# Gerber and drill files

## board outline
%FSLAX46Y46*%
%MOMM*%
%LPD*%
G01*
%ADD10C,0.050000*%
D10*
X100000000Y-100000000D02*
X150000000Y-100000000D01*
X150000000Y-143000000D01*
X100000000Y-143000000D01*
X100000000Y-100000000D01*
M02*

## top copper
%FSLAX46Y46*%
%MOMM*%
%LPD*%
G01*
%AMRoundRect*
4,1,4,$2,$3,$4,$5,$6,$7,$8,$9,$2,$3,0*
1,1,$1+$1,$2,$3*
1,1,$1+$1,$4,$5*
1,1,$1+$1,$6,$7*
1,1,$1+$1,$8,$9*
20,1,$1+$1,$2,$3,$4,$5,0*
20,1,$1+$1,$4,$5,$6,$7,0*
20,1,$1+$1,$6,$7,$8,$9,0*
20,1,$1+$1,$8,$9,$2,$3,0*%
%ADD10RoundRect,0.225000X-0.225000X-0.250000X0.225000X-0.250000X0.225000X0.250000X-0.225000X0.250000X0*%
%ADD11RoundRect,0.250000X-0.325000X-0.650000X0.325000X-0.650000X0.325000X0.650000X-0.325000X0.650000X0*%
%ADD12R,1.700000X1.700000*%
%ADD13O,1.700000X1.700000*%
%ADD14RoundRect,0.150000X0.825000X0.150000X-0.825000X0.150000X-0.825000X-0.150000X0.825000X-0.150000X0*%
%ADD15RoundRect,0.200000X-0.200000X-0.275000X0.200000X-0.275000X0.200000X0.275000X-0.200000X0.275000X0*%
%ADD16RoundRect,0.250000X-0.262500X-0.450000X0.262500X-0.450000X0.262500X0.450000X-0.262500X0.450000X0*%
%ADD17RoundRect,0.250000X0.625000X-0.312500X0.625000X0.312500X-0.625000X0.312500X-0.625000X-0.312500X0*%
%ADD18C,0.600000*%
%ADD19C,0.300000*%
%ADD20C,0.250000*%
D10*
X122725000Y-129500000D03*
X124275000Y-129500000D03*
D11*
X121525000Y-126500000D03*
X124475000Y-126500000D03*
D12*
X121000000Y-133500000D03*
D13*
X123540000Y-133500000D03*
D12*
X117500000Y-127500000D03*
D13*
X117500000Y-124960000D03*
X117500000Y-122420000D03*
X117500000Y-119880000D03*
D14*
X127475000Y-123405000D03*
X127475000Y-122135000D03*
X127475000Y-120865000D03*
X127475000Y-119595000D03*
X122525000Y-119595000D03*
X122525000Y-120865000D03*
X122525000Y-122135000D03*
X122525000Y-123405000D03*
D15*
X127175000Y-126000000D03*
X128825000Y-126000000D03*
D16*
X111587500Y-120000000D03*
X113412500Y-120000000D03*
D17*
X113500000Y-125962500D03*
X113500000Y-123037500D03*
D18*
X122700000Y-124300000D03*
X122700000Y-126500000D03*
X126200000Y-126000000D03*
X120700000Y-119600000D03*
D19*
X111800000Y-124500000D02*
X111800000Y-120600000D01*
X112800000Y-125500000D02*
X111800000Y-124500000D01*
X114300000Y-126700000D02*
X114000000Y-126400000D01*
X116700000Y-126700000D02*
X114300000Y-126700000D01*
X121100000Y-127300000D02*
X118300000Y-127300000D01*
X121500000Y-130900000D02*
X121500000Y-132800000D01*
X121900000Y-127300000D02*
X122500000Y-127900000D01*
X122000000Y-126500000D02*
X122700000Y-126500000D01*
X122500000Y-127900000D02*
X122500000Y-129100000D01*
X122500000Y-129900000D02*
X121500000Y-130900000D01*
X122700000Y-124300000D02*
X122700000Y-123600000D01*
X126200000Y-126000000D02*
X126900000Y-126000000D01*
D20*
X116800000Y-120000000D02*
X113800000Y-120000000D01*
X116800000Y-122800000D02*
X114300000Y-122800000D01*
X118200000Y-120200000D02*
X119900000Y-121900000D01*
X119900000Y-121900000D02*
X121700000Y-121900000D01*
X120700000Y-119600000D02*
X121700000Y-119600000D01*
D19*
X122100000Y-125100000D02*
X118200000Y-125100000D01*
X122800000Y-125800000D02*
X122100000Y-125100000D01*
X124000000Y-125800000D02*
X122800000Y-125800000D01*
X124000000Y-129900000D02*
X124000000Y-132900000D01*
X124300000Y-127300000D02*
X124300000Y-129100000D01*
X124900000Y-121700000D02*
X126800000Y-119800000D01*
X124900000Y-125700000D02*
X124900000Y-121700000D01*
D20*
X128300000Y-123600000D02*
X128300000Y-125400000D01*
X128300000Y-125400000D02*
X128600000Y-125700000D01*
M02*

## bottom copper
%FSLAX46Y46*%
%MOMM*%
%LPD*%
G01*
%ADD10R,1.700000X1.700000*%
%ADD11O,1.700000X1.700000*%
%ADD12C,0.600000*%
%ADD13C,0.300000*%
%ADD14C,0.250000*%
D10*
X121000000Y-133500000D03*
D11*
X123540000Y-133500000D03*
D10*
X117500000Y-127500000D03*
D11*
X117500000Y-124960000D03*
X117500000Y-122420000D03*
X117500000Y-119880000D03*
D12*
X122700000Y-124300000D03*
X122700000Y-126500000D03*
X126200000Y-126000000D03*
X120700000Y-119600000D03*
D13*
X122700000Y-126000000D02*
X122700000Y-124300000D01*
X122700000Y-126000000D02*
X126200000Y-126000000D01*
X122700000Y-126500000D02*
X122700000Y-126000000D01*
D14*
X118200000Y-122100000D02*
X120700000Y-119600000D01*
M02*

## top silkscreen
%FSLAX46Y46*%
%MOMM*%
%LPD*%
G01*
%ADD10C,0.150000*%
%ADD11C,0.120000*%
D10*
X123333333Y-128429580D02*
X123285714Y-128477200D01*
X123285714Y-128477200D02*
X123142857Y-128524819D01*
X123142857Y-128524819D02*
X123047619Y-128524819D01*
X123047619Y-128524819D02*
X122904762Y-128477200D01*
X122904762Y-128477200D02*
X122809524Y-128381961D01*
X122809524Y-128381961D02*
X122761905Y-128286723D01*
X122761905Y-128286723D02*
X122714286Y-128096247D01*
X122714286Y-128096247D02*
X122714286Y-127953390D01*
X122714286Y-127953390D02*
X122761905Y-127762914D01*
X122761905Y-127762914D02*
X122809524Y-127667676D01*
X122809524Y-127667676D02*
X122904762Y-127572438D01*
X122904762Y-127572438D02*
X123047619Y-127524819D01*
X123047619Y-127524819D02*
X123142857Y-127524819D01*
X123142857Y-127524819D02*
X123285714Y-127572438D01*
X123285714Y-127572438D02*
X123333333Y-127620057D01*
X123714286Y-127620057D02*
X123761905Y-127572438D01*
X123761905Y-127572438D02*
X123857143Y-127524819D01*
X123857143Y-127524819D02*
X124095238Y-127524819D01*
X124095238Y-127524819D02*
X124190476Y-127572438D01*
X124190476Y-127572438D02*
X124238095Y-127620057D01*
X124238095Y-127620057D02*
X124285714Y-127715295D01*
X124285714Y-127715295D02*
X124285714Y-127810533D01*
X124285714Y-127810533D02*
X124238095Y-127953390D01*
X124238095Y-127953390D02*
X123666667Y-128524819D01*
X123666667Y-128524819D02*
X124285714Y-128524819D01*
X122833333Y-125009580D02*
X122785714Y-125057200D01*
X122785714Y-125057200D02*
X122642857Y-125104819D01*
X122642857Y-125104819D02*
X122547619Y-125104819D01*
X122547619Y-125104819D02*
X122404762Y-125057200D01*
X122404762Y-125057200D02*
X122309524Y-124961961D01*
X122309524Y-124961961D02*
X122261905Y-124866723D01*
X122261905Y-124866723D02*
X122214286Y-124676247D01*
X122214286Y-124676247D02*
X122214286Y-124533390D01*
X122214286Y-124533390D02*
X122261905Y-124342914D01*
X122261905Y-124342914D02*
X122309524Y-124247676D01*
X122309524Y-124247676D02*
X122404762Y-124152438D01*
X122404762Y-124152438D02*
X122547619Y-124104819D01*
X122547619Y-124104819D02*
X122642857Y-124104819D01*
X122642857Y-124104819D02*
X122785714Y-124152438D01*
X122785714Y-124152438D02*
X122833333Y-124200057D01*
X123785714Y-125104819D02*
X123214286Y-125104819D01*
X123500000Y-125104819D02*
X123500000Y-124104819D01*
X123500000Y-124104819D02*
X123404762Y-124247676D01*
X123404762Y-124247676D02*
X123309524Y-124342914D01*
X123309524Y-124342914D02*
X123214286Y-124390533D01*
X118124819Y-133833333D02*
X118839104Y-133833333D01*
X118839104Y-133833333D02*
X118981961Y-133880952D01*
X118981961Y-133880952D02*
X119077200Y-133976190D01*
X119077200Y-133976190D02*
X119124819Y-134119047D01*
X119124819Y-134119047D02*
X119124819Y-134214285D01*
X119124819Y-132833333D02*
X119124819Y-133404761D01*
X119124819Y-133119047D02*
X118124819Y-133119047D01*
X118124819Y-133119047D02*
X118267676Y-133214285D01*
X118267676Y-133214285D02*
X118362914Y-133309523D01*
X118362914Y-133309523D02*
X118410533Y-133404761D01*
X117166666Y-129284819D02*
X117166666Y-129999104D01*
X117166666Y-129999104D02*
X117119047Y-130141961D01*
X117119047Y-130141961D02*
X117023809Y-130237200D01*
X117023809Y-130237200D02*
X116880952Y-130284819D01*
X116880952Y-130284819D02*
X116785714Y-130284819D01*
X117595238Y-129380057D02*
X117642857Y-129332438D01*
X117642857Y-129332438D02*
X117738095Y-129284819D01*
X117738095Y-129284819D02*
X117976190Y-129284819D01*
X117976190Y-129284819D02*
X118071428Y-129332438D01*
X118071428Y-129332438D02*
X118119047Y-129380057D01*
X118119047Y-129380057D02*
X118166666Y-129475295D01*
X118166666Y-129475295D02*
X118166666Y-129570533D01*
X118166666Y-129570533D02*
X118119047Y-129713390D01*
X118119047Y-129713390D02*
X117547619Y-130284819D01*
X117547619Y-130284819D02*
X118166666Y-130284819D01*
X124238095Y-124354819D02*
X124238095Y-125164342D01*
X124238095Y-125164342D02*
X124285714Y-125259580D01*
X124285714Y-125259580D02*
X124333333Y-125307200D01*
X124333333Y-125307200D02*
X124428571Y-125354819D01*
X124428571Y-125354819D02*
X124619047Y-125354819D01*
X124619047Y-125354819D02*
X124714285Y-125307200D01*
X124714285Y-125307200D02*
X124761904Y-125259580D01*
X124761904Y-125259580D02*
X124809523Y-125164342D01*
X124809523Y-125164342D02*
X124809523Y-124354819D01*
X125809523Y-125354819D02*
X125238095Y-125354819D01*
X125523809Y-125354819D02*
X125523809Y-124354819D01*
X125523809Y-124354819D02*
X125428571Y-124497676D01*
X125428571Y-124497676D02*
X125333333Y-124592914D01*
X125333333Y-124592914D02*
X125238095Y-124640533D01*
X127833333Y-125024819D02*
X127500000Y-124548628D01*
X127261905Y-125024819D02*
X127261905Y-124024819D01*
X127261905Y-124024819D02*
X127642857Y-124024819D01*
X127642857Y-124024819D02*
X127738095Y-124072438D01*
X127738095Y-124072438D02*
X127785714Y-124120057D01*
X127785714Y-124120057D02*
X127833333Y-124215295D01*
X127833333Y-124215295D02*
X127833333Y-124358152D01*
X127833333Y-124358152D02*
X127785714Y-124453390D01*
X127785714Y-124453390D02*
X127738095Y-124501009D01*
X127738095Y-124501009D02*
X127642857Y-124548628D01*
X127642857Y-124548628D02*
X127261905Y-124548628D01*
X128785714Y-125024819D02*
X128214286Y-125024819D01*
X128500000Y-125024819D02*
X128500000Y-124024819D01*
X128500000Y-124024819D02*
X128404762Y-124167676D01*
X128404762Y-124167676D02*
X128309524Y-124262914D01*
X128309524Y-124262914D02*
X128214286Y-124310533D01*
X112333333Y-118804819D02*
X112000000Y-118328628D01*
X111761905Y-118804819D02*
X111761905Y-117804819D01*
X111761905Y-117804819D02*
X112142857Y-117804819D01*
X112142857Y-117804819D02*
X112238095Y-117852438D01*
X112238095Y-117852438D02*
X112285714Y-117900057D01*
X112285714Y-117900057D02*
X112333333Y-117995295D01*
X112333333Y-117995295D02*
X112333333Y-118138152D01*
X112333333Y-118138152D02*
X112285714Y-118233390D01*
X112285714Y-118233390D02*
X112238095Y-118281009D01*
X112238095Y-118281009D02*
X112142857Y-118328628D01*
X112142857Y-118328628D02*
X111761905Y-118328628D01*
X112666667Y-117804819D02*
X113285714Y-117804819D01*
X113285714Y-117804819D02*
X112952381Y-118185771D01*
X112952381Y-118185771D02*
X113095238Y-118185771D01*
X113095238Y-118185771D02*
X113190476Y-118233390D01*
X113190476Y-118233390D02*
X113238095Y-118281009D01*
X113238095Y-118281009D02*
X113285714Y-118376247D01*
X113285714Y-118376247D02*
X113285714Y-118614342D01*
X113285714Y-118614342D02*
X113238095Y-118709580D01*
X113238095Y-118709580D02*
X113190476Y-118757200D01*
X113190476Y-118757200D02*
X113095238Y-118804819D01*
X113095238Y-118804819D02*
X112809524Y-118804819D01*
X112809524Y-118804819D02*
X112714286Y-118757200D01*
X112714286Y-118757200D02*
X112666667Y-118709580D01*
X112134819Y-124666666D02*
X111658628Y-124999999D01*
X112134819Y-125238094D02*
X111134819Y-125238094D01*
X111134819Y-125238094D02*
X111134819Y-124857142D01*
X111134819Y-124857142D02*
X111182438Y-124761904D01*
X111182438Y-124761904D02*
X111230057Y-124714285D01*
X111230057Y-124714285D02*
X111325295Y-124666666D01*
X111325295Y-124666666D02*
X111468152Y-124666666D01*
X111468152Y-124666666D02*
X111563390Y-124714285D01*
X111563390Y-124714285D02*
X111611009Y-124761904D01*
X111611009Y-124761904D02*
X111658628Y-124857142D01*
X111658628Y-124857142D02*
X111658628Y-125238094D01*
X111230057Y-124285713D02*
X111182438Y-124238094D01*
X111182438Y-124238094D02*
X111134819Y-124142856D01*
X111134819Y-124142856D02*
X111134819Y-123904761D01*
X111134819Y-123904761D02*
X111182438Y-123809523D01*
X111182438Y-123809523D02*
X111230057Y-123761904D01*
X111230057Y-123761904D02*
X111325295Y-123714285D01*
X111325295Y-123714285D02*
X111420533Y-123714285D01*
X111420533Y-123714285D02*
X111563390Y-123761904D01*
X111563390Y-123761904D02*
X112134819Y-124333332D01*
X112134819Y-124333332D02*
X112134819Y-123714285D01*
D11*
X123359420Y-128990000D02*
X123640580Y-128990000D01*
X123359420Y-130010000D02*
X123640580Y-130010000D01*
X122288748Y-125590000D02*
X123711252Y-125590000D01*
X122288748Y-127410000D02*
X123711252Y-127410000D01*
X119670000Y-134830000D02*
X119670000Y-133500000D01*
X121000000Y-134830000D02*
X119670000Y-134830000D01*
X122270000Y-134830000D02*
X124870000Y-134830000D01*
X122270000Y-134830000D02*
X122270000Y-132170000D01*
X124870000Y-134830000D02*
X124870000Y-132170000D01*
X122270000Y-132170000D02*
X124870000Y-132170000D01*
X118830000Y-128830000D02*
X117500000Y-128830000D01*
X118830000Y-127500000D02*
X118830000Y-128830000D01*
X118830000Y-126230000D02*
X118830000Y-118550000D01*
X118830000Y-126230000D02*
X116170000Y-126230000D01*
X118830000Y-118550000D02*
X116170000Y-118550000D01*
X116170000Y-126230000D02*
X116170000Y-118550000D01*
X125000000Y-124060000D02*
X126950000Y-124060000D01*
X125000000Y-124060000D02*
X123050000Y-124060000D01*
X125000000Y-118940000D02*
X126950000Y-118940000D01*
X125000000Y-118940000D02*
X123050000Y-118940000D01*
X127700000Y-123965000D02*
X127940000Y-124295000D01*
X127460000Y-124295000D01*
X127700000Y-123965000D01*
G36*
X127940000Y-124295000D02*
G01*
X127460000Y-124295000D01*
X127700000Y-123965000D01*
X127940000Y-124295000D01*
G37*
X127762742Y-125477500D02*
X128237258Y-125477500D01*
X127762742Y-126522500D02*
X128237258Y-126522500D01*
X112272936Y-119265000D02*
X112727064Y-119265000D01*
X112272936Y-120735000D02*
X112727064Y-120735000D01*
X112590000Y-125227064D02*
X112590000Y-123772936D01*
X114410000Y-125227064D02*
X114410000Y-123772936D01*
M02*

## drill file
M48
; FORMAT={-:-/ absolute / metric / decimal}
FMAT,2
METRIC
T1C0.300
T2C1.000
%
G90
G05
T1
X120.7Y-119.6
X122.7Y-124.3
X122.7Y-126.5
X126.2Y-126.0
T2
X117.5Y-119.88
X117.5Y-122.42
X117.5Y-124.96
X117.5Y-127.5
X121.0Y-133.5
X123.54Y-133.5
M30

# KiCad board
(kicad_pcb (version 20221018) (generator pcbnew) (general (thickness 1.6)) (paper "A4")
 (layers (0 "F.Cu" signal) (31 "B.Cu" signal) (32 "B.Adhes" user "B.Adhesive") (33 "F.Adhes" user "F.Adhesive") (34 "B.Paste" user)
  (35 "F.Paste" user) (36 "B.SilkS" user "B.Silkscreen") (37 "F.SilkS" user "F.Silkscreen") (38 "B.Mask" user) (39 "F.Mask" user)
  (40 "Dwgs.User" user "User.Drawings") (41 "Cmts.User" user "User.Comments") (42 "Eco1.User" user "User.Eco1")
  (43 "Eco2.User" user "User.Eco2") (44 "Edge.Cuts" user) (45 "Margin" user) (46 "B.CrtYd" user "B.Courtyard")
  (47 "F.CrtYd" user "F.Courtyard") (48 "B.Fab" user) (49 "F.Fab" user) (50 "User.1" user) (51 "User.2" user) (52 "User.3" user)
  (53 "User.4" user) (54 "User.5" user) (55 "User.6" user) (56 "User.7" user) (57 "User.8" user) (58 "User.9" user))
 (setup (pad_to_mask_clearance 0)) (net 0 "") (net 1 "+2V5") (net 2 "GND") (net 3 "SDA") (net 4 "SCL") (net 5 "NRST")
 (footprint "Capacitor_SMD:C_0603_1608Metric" (layer "F.Cu") (at 123.5 129.5)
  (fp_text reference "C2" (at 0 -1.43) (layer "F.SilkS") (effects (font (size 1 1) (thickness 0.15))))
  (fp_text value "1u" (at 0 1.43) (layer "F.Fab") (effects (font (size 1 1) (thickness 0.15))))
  (fp_line (start -0.14058 -0.51) (end 0.14058 -0.51) (stroke (width 0.12) (type solid)) (layer "F.SilkS"))
  (fp_line (start -0.14058 0.51) (end 0.14058 0.51) (stroke (width 0.12) (type solid)) (layer "F.SilkS"))
  (pad "1" smd roundrect (at -0.775 0) (size 0.9 0.95) (layers "F.Cu" "F.Paste" "F.Mask") (roundrect_rratio 0.25) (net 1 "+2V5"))
  (pad "2" smd roundrect (at 0.775 0) (size 0.9 0.95) (layers "F.Cu" "F.Paste" "F.Mask") (roundrect_rratio 0.25) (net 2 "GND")))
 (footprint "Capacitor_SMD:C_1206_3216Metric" (layer "F.Cu") (at 123 126.5)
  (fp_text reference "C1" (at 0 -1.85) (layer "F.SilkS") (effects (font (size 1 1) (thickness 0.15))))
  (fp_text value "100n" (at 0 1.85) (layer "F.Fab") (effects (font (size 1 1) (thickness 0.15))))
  (fp_line (start -0.711252 -0.91) (end 0.711252 -0.91) (stroke (width 0.12) (type solid)) (layer "F.SilkS"))
  (fp_line (start -0.711252 0.91) (end 0.711252 0.91) (stroke (width 0.12) (type solid)) (layer "F.SilkS"))
  (pad "1" smd roundrect (at -1.475 0) (size 1.15 1.8) (layers "F.Cu" "F.Paste" "F.Mask") (roundrect_rratio 0.217391) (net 1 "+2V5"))
  (pad "2" smd roundrect (at 1.475 0) (size 1.15 1.8) (layers "F.Cu" "F.Paste" "F.Mask") (roundrect_rratio 0.217391) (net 2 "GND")))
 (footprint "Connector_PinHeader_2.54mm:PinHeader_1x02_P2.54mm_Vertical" (layer "F.Cu") (at 121 133.5 90)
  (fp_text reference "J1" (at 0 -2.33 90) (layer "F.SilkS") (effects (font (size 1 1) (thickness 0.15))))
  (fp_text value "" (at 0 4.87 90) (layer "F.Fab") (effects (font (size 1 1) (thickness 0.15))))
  (fp_line (start -1.33 -1.33) (end 0 -1.33) (stroke (width 0.12) (type solid)) (layer "F.SilkS"))
  (fp_line (start -1.33 0) (end -1.33 -1.33) (stroke (width 0.12) (type solid)) (layer "F.SilkS"))
  (fp_line (start -1.33 1.27) (end -1.33 3.87) (stroke (width 0.12) (type solid)) (layer "F.SilkS"))
  (fp_line (start -1.33 1.27) (end 1.33 1.27) (stroke (width 0.12) (type solid)) (layer "F.SilkS"))
  (fp_line (start -1.33 3.87) (end 1.33 3.87) (stroke (width 0.12) (type solid)) (layer "F.SilkS"))
  (fp_line (start 1.33 1.27) (end 1.33 3.87) (stroke (width 0.12) (type solid)) (layer "F.SilkS"))
  (pad "1" thru_hole rect (at 0 0 90) (size 1.7 1.7) (drill 1) (layers "*.Cu" "*.Mask") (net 1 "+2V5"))
  (pad "2" thru_hole oval (at 0 2.54 90) (size 1.7 1.7) (drill 1) (layers "*.Cu" "*.Mask") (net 2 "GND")))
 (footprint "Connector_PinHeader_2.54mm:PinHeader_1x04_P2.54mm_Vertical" (layer "F.Cu") (at 117.5 127.5 180)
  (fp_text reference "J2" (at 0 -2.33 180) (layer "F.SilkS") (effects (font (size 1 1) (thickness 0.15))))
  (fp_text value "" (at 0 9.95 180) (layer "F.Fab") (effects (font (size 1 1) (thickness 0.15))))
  (fp_line (start -1.33 -1.33) (end 0 -1.33) (stroke (width 0.12) (type solid)) (layer "F.SilkS"))
  (fp_line (start -1.33 0) (end -1.33 -1.33) (stroke (width 0.12) (type solid)) (layer "F.SilkS"))
  (fp_line (start -1.33 1.27) (end -1.33 8.95) (stroke (width 0.12) (type solid)) (layer "F.SilkS"))
  (fp_line (start -1.33 1.27) (end 1.33 1.27) (stroke (width 0.12) (type solid)) (layer "F.SilkS"))
  (fp_line (start -1.33 8.95) (end 1.33 8.95) (stroke (width 0.12) (type solid)) (layer "F.SilkS"))
  (fp_line (start 1.33 1.27) (end 1.33 8.95) (stroke (width 0.12) (type solid)) (layer "F.SilkS"))
  (pad "1" thru_hole rect (at 0 0 180) (size 1.7 1.7) (drill 1) (layers "*.Cu" "*.Mask") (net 1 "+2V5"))
  (pad "2" thru_hole oval (at 0 2.54 180) (size 1.7 1.7) (drill 1) (layers "*.Cu" "*.Mask") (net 2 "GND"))
  (pad "3" thru_hole oval (at 0 5.08 180) (size 1.7 1.7) (drill 1) (layers "*.Cu" "*.Mask") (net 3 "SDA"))
  (pad "4" thru_hole oval (at 0 7.62 180) (size 1.7 1.7) (drill 1) (layers "*.Cu" "*.Mask") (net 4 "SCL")))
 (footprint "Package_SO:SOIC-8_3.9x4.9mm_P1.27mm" (layer "F.Cu") (at 125 121.5 180)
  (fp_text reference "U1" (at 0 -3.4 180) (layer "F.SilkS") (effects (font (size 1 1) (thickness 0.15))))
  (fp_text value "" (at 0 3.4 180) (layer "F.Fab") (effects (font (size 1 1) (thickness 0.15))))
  (fp_line (start 0 -2.56) (end -1.95 -2.56) (stroke (width 0.12) (type solid)) (layer "F.SilkS"))
  (fp_line (start 0 -2.56) (end 1.95 -2.56) (stroke (width 0.12) (type solid)) (layer "F.SilkS"))
  (fp_line (start 0 2.56) (end -1.95 2.56) (stroke (width 0.12) (type solid)) (layer "F.SilkS"))
  (fp_line (start 0 2.56) (end 1.95 2.56) (stroke (width 0.12) (type solid)) (layer "F.SilkS"))
  (fp_poly
   (pts (xy -2.7 -2.465) (xy -2.94 -2.795) (xy -2.46 -2.795) (xy -2.7 -2.465)) (stroke (width 0.12) (type solid)) (fill solid)
   (layer "F.SilkS"))
  (pad "1" smd roundrect (at -2.475 -1.905 180) (size 1.95 0.6) (layers "F.Cu" "F.Paste" "F.Mask") (roundrect_rratio 0.25) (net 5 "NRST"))
  (pad "2" smd roundrect (at -2.475 -0.635 180) (size 1.95 0.6) (layers "F.Cu" "F.Paste" "F.Mask") (roundrect_rratio 0.25))
  (pad "3" smd roundrect (at -2.475 0.635 180) (size 1.95 0.6) (layers "F.Cu" "F.Paste" "F.Mask") (roundrect_rratio 0.25))
  (pad "4" smd roundrect (at -2.475 1.905 180) (size 1.95 0.6) (layers "F.Cu" "F.Paste" "F.Mask") (roundrect_rratio 0.25) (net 2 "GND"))
  (pad "5" smd roundrect (at 2.475 1.905 180) (size 1.95 0.6) (layers "F.Cu" "F.Paste" "F.Mask") (roundrect_rratio 0.25) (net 3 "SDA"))
  (pad "6" smd roundrect (at 2.475 0.635 180) (size 1.95 0.6) (layers "F.Cu" "F.Paste" "F.Mask") (roundrect_rratio 0.25))
  (pad "7" smd roundrect (at 2.475 -0.635 180) (size 1.95 0.6) (layers "F.Cu" "F.Paste" "F.Mask") (roundrect_rratio 0.25) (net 4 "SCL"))
  (pad "8" smd roundrect (at 2.475 -1.905 180) (size 1.95 0.6) (layers "F.Cu" "F.Paste" "F.Mask") (roundrect_rratio 0.25) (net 1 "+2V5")))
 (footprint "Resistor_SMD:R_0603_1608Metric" (layer "F.Cu") (at 128 126)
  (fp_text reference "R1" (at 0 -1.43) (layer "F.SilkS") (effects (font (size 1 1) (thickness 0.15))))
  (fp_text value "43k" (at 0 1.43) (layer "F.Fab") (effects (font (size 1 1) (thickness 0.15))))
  (fp_line (start -0.237258 -0.5225) (end 0.237258 -0.5225) (stroke (width 0.12) (type solid)) (layer "F.SilkS"))
  (fp_line (start -0.237258 0.5225) (end 0.237258 0.5225) (stroke (width 0.12) (type solid)) (layer "F.SilkS"))
  (pad "1" smd roundrect (at -0.825 0) (size 0.8 0.95) (layers "F.Cu" "F.Paste" "F.Mask") (roundrect_rratio 0.25) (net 1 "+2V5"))
  (pad "2" smd roundrect (at 0.825 0) (size 0.8 0.95) (layers "F.Cu" "F.Paste" "F.Mask") (roundrect_rratio 0.25) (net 5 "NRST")))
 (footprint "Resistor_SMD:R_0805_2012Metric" (layer "F.Cu") (at 112.5 120)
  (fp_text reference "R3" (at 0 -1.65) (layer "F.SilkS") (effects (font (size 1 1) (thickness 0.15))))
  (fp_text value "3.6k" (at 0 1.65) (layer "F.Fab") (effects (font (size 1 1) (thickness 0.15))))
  (fp_line (start -0.227064 -0.735) (end 0.227064 -0.735) (stroke (width 0.12) (type solid)) (layer "F.SilkS"))
  (fp_line (start -0.227064 0.735) (end 0.227064 0.735) (stroke (width 0.12) (type solid)) (layer "F.SilkS"))
  (pad "1" smd roundrect (at -0.9125 0) (size 1.025 1.4) (layers "F.Cu" "F.Paste" "F.Mask") (roundrect_rratio 0.243902) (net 1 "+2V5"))
  (pad "2" smd roundrect (at 0.9125 0) (size 1.025 1.4) (layers "F.Cu" "F.Paste" "F.Mask") (roundrect_rratio 0.243902) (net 4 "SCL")))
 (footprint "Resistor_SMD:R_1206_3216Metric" (layer "F.Cu") (at 113.5 124.5 90)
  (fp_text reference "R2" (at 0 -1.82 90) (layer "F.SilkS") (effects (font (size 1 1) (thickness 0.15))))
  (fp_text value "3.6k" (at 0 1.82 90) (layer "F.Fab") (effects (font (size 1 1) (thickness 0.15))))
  (fp_line (start -0.727064 -0.91) (end 0.727064 -0.91) (stroke (width 0.12) (type solid)) (layer "F.SilkS"))
  (fp_line (start -0.727064 0.91) (end 0.727064 0.91) (stroke (width 0.12) (type solid)) (layer "F.SilkS"))
  (pad "1" smd roundrect (at -1.4625 0 90) (size 1.125 1.75) (layers "F.Cu" "F.Paste" "F.Mask") (roundrect_rratio 0.222222) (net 1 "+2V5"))
  (pad "2" smd roundrect (at 1.4625 0 90) (size 1.125 1.75) (layers "F.Cu" "F.Paste" "F.Mask") (roundrect_rratio 0.222222) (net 3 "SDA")))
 (gr_rect (start 100 100) (end 150 143) (stroke (width 0.05) (type default)) (fill none) (layer "Edge.Cuts"))
 (segment (start 111.8 124.5) (end 111.8 120.6) (width 0.3) (layer "F.Cu") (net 1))
 (segment (start 112.8 125.5) (end 111.8 124.5) (width 0.3) (layer "F.Cu") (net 1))
 (segment (start 114.3 126.7) (end 114 126.4) (width 0.3) (layer "F.Cu") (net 1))
 (segment (start 116.7 126.7) (end 114.3 126.7) (width 0.3) (layer "F.Cu") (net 1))
 (segment (start 121.1 127.3) (end 118.3 127.3) (width 0.3) (layer "F.Cu") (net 1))
 (segment (start 121.5 130.9) (end 121.5 132.8) (width 0.3) (layer "F.Cu") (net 1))
 (segment (start 121.9 127.3) (end 122.5 127.9) (width 0.3) (layer "F.Cu") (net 1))
 (segment (start 122 126.5) (end 122.7 126.5) (width 0.3) (layer "F.Cu") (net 1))
 (segment (start 122.5 127.9) (end 122.5 129.1) (width 0.3) (layer "F.Cu") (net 1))
 (segment (start 122.5 129.9) (end 121.5 130.9) (width 0.3) (layer "F.Cu") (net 1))
 (segment (start 122.7 124.3) (end 122.7 123.6) (width 0.3) (layer "F.Cu") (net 1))
 (segment (start 126.2 126) (end 126.9 126) (width 0.3) (layer "F.Cu") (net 1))
 (via (at 122.7 124.3) (size 0.6) (drill 0.3) (layers "F.Cu" "B.Cu") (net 1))
 (via (at 122.7 126.5) (size 0.6) (drill 0.3) (layers "F.Cu" "B.Cu") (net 1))
 (via (at 126.2 126) (size 0.6) (drill 0.3) (layers "F.Cu" "B.Cu") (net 1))
 (segment (start 116.8 120) (end 113.8 120) (width 0.25) (layer "F.Cu") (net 4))
 (segment (start 116.8 122.8) (end 114.3 122.8) (width 0.25) (layer "F.Cu") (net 3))
 (segment (start 118.2 120.2) (end 119.9 121.9) (width 0.25) (layer "F.Cu") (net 4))
 (segment (start 119.9 121.9) (end 121.7 121.9) (width 0.25) (layer "F.Cu") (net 4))
 (segment (start 120.7 119.6) (end 121.7 119.6) (width 0.25) (layer "F.Cu") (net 3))
 (segment (start 122.1 125.1) (end 118.2 125.1) (width 0.3) (layer "F.Cu") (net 2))
 (segment (start 122.7 126) (end 122.7 124.3) (width 0.3) (layer "B.Cu") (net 1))
 (segment (start 122.7 126) (end 126.2 126) (width 0.3) (layer "B.Cu") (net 1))
 (segment (start 122.7 126.5) (end 122.7 126) (width 0.3) (layer "B.Cu") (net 1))
 (segment (start 122.8 125.8) (end 122.1 125.1) (width 0.3) (layer "F.Cu") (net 2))
 (segment (start 124 125.8) (end 122.8 125.8) (width 0.3) (layer "F.Cu") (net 2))
 (segment (start 124 129.9) (end 124 132.9) (width 0.3) (layer "F.Cu") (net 2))
 (segment (start 124.3 127.3) (end 124.3 129.1) (width 0.3) (layer "F.Cu") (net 2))
 (segment (start 124.9 121.7) (end 126.8 119.8) (width 0.3) (layer "F.Cu") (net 2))
 (segment (start 124.9 125.7) (end 124.9 121.7) (width 0.3) (layer "F.Cu") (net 2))
 (segment (start 128.3 123.6) (end 128.3 125.4) (width 0.25) (layer "F.Cu") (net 5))
 (segment (start 128.3 125.4) (end 128.6 125.7) (width 0.25) (layer "F.Cu") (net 5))
 (via (at 120.7 119.6) (size 0.6) (drill 0.3) (layers "F.Cu" "B.Cu") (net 3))
 (segment (start 118.2 122.1) (end 120.7 119.6) (width 0.25) (layer "B.Cu") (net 3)))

